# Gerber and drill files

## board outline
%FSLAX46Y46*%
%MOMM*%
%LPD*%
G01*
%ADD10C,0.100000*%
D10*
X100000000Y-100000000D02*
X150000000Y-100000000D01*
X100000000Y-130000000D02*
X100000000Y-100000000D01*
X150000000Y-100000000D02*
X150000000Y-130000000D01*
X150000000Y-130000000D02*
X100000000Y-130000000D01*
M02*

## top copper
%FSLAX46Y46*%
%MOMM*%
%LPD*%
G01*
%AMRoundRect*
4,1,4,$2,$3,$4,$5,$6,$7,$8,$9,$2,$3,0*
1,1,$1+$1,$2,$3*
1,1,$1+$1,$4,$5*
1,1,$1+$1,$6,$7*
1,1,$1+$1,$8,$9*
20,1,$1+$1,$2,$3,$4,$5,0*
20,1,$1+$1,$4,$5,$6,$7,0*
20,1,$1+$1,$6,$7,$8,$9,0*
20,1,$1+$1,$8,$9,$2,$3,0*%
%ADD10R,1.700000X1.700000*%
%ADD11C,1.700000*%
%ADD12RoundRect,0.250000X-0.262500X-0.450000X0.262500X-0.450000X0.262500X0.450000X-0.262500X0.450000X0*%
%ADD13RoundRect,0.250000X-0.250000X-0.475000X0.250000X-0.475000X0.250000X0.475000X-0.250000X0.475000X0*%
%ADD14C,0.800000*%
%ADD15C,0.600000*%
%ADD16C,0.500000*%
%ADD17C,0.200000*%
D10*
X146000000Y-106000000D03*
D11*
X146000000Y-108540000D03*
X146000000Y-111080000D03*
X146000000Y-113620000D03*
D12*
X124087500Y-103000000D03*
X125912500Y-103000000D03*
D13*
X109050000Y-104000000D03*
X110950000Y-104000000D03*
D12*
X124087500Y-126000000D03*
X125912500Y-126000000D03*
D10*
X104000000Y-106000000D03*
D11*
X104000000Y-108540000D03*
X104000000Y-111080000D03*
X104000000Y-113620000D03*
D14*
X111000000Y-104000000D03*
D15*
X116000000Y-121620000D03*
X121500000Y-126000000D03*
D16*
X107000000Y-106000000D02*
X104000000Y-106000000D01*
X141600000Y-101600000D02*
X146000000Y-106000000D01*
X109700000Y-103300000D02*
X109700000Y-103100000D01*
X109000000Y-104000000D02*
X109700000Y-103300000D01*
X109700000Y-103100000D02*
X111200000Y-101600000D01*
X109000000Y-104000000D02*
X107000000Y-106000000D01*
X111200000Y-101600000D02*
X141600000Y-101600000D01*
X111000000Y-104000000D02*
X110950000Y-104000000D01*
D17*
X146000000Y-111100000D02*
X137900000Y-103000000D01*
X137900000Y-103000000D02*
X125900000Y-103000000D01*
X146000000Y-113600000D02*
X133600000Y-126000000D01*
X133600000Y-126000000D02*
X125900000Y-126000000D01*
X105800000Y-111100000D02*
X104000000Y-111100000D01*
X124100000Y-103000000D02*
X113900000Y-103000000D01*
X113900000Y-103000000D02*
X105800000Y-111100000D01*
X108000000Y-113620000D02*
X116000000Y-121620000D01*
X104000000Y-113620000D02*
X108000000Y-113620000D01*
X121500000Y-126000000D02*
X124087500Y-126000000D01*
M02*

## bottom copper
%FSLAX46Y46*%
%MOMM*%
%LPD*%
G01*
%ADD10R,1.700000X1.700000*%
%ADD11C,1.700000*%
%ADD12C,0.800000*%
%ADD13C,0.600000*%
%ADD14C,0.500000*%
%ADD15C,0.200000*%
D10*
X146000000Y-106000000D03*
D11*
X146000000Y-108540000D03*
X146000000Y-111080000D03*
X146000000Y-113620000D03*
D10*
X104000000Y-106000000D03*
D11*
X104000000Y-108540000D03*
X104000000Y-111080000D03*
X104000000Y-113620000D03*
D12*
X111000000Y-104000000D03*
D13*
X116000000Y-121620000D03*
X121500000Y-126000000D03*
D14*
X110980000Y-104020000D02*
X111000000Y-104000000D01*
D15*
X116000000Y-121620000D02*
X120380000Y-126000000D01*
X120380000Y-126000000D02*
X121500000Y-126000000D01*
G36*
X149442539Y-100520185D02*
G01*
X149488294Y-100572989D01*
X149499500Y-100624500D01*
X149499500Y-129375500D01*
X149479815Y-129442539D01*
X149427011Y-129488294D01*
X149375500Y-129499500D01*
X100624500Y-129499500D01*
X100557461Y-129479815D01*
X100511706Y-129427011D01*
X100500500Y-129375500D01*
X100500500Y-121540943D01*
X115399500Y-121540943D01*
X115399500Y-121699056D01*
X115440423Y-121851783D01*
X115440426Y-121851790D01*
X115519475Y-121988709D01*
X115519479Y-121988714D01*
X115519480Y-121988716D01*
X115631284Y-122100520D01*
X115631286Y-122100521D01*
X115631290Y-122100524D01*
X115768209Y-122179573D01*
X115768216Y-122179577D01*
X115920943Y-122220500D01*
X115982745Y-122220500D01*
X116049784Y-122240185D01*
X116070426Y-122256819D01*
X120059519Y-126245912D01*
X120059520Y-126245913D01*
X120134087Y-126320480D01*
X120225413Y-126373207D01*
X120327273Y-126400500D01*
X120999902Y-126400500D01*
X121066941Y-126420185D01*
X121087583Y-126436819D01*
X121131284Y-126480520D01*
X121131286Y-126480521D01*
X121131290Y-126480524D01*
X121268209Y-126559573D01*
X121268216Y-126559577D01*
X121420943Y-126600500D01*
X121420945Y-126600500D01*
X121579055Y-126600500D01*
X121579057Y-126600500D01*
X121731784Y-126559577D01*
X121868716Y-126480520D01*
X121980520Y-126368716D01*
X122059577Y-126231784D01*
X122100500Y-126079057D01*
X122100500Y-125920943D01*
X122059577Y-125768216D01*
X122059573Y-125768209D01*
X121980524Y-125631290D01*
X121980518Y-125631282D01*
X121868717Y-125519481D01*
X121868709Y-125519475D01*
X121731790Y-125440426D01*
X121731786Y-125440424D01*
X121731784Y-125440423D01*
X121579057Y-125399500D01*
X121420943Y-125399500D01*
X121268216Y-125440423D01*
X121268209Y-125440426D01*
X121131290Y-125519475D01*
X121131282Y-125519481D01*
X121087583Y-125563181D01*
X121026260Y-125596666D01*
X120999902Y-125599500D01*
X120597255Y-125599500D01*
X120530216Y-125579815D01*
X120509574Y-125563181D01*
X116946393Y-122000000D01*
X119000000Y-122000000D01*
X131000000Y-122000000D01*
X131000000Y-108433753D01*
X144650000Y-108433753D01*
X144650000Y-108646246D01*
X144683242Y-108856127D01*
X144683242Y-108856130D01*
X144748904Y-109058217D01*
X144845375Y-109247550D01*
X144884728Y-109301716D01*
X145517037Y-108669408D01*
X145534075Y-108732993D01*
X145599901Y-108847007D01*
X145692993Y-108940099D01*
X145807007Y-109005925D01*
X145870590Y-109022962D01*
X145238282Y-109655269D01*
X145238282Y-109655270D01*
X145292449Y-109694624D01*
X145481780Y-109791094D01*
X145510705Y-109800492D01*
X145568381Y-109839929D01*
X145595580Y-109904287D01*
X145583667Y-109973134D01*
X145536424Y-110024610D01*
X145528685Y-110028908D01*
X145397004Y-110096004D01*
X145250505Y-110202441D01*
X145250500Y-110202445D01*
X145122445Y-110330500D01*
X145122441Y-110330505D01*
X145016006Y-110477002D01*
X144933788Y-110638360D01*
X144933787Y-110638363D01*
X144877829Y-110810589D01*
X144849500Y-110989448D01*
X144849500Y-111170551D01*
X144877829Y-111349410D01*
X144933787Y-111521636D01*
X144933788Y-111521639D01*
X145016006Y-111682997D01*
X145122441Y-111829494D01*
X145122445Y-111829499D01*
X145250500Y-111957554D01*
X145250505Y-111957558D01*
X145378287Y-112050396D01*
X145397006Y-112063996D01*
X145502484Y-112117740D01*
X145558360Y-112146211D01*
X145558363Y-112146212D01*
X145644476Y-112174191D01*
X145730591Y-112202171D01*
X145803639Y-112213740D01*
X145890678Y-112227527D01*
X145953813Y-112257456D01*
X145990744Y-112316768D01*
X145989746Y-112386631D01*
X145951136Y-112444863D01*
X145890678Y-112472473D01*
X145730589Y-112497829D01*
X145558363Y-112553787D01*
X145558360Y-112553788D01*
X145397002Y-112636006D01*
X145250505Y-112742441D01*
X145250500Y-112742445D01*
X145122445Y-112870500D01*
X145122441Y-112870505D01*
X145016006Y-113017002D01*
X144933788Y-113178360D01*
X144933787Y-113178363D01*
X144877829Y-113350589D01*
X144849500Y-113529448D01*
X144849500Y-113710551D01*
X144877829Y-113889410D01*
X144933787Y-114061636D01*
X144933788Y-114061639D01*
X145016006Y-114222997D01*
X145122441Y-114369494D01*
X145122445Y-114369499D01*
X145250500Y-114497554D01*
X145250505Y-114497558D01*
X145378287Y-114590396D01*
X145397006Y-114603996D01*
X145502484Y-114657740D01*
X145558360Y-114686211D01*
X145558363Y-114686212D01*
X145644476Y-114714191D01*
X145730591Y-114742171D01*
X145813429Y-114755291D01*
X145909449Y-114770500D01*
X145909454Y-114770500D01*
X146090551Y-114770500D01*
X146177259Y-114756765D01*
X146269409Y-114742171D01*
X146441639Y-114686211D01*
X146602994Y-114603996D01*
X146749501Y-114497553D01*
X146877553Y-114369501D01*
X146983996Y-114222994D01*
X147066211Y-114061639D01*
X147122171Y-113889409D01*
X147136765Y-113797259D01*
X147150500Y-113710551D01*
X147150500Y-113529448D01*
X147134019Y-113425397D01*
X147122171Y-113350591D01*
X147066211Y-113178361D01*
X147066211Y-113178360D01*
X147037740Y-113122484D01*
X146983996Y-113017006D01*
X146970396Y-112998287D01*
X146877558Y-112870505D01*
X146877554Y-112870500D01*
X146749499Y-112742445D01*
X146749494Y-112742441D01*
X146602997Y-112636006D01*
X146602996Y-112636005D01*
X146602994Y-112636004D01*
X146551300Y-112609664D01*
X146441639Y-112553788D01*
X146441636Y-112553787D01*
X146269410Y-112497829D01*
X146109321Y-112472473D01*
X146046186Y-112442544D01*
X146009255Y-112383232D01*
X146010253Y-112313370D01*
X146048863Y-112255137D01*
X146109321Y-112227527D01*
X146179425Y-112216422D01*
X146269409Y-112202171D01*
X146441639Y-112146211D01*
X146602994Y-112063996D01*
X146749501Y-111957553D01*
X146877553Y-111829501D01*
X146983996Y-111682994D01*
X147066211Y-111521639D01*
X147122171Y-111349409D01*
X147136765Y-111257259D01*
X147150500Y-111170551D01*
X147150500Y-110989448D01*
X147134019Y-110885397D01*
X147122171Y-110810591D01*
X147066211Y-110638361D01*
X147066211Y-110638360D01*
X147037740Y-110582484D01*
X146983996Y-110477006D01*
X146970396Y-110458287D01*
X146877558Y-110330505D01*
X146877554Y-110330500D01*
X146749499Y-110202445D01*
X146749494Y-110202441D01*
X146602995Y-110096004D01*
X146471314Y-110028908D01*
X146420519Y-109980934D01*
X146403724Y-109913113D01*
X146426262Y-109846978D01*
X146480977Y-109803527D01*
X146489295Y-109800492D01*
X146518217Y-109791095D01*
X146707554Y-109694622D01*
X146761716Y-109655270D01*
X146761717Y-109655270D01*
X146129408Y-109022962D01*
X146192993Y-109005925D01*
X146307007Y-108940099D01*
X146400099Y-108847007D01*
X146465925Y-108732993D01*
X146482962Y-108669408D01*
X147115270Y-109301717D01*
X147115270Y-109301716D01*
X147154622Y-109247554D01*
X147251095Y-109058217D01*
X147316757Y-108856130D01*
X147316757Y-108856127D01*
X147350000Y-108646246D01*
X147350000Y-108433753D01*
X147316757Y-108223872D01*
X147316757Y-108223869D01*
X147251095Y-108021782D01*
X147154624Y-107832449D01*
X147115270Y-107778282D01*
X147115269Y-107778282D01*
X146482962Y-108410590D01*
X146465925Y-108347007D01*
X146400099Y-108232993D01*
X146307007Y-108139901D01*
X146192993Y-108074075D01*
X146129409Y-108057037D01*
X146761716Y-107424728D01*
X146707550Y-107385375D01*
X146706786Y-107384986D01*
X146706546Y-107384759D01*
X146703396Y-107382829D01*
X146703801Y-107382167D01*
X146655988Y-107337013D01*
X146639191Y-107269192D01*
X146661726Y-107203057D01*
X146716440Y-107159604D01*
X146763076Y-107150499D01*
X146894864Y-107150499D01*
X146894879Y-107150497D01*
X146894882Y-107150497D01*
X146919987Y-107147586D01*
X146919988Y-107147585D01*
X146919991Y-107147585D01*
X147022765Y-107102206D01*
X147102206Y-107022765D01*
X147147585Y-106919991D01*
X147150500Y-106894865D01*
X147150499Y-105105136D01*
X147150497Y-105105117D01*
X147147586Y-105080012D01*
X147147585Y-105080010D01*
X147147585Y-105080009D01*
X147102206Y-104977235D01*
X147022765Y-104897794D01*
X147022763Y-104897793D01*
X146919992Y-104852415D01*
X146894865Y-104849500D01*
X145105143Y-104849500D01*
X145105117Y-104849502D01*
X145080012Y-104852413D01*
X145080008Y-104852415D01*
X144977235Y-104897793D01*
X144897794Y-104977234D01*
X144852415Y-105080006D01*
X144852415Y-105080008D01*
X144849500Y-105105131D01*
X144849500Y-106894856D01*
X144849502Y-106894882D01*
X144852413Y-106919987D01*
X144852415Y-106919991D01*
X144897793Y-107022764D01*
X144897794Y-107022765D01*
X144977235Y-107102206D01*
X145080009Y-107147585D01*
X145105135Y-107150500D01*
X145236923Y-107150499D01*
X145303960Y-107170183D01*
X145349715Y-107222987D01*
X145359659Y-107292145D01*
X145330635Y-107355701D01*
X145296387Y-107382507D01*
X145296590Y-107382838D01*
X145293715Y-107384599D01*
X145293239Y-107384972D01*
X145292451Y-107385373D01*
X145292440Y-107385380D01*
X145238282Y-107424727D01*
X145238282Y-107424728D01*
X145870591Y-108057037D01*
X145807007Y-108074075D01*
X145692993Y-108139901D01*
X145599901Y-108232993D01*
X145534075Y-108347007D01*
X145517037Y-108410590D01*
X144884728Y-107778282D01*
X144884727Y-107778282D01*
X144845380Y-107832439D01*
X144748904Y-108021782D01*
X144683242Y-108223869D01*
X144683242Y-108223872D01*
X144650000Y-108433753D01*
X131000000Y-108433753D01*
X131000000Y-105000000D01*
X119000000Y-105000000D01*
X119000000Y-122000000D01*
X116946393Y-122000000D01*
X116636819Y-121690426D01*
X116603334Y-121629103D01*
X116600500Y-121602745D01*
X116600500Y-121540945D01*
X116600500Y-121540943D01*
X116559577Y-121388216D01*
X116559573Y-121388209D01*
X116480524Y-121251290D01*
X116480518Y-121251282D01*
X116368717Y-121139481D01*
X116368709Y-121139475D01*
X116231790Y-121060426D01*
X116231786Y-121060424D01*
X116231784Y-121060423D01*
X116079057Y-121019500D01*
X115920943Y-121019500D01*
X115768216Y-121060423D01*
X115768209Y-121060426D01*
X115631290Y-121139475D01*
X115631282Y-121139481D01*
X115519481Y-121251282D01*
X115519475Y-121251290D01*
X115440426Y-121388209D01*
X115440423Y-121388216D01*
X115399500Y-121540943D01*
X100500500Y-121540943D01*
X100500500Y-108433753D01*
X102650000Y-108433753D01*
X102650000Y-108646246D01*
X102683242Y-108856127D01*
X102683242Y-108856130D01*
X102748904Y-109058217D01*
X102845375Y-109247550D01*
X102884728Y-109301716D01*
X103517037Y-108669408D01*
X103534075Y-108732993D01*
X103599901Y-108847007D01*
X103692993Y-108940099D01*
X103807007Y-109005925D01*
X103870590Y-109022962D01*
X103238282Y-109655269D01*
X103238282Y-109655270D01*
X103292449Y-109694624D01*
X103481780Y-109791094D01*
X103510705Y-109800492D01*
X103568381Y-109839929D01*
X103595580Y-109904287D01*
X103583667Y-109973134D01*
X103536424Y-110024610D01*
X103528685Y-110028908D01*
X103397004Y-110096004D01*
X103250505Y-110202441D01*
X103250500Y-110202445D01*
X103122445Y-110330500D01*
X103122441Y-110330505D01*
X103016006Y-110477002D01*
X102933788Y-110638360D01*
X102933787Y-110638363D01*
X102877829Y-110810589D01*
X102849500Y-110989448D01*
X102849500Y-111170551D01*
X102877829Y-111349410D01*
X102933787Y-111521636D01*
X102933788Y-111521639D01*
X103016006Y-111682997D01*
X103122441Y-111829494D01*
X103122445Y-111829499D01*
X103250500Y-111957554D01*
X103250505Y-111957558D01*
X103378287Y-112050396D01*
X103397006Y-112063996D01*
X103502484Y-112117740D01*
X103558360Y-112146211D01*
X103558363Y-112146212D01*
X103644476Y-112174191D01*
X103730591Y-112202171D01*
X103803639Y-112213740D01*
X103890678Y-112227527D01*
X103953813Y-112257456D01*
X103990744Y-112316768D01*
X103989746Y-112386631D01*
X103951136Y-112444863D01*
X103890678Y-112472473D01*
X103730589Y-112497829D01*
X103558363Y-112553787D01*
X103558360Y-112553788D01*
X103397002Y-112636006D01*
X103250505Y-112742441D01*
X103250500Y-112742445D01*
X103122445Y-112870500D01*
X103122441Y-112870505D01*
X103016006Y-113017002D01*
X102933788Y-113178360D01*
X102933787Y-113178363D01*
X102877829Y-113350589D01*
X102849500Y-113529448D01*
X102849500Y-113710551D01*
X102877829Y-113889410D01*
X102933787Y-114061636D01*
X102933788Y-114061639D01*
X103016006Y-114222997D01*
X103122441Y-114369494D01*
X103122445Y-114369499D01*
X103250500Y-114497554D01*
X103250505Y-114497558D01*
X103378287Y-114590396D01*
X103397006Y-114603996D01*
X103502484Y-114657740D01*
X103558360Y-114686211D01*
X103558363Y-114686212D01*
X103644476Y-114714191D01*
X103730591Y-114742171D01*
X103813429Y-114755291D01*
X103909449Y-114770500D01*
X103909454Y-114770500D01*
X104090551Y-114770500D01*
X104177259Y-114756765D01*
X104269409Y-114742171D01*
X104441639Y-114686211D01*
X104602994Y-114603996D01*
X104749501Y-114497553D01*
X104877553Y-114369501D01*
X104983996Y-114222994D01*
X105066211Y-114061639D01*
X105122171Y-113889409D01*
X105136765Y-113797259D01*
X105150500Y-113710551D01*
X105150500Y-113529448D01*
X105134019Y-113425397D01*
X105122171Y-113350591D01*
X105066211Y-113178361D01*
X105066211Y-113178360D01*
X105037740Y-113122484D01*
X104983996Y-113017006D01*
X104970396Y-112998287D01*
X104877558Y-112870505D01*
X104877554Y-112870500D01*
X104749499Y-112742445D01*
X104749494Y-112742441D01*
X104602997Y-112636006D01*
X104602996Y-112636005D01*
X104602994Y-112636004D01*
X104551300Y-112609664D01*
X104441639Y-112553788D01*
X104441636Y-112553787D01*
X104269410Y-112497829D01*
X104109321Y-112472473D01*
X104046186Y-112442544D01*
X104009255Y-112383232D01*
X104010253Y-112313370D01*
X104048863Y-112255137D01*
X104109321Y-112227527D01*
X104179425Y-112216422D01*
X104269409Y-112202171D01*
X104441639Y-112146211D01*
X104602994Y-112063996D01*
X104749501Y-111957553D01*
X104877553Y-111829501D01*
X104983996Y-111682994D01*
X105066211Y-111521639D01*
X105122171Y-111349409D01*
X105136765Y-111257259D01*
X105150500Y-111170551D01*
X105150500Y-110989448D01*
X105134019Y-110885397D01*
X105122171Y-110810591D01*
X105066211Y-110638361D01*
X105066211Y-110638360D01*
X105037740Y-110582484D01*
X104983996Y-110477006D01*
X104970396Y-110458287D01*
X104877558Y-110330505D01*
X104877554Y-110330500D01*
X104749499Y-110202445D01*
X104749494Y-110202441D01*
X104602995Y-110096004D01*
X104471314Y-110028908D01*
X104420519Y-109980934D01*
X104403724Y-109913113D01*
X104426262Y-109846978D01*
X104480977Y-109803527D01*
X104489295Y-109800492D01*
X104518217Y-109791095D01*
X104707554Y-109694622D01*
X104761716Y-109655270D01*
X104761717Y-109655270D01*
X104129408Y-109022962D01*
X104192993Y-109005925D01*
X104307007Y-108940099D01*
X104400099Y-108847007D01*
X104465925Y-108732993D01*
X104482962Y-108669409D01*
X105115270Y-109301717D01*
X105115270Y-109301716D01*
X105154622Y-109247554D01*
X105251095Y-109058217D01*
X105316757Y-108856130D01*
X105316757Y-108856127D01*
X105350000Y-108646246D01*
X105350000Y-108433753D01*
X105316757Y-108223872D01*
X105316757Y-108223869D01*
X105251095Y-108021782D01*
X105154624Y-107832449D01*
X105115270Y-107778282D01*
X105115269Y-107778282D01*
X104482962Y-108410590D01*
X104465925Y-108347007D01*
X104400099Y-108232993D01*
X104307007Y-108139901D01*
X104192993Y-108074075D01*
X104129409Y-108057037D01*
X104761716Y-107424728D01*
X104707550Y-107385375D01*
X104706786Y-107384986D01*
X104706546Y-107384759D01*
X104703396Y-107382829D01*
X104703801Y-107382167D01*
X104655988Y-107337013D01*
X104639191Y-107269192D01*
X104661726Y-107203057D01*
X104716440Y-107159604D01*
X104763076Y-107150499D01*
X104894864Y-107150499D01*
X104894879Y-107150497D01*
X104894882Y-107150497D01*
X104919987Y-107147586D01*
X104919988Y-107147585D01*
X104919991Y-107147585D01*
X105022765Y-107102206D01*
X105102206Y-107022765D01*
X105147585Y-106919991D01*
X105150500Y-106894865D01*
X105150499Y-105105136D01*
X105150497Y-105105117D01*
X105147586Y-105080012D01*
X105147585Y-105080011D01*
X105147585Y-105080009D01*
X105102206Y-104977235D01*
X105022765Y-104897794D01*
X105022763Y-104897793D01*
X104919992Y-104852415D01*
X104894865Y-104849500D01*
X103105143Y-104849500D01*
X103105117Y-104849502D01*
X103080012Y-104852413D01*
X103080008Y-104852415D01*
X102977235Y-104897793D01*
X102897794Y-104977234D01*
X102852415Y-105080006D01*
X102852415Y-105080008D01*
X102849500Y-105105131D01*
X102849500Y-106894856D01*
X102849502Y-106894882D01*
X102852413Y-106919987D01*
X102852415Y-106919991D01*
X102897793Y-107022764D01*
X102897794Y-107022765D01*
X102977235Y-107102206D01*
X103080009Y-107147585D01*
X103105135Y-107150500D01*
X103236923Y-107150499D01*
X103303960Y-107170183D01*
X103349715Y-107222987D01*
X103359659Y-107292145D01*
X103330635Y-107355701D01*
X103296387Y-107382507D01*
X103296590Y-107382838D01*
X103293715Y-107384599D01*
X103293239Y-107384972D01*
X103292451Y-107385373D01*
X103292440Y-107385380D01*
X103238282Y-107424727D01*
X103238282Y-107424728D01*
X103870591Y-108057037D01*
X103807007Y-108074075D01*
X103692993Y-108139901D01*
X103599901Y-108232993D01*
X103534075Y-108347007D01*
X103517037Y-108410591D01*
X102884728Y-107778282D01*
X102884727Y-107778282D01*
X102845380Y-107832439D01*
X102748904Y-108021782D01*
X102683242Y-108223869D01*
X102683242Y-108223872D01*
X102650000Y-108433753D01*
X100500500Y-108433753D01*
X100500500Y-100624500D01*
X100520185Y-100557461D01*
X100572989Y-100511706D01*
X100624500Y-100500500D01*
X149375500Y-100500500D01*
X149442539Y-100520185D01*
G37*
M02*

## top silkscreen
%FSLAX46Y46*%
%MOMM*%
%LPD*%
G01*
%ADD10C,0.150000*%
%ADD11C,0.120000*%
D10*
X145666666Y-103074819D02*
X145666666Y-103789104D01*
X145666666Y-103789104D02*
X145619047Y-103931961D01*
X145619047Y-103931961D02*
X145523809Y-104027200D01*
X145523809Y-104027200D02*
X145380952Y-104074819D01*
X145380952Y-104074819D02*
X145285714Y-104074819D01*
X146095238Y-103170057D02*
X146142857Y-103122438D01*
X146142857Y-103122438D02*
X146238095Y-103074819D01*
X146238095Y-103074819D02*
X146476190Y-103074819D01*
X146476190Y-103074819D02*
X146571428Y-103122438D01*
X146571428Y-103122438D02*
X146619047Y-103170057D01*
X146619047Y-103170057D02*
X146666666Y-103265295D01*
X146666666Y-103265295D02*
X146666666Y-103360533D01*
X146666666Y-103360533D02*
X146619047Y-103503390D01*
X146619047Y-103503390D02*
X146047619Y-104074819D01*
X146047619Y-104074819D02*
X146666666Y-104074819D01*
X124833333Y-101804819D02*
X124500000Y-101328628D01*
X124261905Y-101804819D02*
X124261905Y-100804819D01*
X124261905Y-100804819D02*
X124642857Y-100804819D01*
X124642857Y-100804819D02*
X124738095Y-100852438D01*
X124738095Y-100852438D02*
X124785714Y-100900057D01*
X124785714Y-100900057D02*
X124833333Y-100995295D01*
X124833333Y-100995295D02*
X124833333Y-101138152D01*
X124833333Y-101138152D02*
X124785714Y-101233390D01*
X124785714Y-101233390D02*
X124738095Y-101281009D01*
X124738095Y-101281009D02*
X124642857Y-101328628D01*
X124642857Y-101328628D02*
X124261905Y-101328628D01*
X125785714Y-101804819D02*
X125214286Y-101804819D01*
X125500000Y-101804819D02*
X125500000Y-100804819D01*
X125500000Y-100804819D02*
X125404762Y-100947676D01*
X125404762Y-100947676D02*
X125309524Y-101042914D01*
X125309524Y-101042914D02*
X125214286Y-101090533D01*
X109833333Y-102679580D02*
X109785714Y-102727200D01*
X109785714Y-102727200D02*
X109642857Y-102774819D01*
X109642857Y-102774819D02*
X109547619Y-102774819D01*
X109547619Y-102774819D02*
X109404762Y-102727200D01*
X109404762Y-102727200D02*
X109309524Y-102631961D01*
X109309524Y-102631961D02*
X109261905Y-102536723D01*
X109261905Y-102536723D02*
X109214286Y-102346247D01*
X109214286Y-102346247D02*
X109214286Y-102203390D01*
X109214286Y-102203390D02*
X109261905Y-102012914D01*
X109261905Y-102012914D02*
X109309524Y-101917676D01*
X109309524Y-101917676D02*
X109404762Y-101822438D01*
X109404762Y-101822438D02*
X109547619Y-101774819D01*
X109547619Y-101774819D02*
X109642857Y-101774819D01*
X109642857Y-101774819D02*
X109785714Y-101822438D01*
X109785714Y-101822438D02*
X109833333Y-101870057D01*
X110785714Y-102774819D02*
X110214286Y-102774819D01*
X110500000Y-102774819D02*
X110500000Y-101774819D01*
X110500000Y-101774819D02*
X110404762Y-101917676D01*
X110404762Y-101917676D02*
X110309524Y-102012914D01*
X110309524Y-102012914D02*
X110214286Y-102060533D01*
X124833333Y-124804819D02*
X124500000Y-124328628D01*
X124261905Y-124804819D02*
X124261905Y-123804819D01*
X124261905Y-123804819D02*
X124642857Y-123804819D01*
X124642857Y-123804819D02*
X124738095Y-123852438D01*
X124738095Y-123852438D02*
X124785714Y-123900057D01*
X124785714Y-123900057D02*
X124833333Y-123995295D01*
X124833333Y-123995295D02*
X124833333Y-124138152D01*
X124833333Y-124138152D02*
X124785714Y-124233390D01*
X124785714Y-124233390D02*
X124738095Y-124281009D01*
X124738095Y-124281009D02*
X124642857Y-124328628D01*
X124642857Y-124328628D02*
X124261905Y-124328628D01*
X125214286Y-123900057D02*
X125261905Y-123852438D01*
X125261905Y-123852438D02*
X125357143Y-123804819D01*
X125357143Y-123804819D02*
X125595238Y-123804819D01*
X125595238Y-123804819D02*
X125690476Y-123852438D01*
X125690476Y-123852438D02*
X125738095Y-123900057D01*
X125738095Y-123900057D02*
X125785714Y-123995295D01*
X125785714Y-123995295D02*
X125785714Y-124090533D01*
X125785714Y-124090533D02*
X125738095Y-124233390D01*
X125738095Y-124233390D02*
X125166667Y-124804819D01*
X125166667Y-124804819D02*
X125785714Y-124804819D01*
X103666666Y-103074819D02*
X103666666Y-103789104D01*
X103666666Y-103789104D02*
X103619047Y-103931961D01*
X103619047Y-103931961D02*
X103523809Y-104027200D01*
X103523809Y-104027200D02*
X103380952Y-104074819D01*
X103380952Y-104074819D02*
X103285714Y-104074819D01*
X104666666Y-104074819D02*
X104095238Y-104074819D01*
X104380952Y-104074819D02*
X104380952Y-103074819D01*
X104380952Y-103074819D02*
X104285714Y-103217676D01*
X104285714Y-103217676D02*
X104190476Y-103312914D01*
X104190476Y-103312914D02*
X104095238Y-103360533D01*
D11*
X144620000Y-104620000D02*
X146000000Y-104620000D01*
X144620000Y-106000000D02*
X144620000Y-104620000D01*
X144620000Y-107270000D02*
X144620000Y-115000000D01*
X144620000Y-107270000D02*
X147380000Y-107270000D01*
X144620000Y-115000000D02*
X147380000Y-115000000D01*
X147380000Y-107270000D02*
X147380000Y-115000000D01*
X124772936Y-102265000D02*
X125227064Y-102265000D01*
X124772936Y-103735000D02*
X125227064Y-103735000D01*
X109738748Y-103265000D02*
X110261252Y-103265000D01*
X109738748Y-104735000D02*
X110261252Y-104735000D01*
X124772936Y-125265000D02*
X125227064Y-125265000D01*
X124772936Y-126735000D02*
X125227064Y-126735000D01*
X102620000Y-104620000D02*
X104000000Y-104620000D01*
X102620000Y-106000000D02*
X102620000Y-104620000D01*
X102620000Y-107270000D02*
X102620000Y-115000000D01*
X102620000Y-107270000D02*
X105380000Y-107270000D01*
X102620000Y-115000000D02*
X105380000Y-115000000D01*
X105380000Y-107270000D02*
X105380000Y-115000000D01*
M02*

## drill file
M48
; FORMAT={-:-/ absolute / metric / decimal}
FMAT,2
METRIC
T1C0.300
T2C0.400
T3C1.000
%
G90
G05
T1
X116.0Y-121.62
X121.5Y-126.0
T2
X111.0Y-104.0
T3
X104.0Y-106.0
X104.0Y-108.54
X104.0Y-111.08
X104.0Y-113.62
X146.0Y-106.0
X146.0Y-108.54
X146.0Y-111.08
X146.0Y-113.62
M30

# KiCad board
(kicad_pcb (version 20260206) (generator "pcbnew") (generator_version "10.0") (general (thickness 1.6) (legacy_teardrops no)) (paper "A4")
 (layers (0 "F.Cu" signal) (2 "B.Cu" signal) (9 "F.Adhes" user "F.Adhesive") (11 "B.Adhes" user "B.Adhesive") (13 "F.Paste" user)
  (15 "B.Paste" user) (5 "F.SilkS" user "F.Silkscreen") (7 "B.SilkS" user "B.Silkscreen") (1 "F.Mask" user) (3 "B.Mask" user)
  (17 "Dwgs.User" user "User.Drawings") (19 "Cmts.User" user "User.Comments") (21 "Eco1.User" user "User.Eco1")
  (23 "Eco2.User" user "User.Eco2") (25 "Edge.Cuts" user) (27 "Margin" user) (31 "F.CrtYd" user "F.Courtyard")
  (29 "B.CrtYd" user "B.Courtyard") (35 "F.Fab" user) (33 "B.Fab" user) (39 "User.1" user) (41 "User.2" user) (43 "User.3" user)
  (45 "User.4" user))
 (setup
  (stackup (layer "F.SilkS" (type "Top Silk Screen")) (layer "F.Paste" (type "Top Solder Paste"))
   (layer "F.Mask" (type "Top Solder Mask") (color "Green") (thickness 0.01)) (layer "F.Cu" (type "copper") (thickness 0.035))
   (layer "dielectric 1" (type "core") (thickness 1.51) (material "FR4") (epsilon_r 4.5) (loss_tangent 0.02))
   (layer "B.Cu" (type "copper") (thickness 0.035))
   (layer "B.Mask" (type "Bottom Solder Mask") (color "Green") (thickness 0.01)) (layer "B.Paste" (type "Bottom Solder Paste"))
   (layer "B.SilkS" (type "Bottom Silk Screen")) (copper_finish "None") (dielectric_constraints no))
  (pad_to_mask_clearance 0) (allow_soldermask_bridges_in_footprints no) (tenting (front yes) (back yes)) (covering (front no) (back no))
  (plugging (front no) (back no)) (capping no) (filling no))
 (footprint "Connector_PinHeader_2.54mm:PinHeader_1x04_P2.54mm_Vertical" (layer "F.Cu") (at 146 106)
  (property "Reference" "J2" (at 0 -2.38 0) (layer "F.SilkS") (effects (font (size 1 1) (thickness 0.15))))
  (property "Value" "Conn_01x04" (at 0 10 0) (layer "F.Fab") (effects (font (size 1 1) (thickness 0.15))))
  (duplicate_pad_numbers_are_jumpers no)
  (fp_line (start -1.38 -1.38) (end 0 -1.38) (stroke (width 0.12) (type solid)) (layer "F.SilkS"))
  (fp_line (start -1.38 0) (end -1.38 -1.38) (stroke (width 0.12) (type solid)) (layer "F.SilkS"))
  (fp_line (start -1.38 1.27) (end -1.38 9) (stroke (width 0.12) (type solid)) (layer "F.SilkS"))
  (fp_line (start -1.38 1.27) (end 1.38 1.27) (stroke (width 0.12) (type solid)) (layer "F.SilkS"))
  (fp_line (start -1.38 9) (end 1.38 9) (stroke (width 0.12) (type solid)) (layer "F.SilkS"))
  (fp_line (start 1.38 1.27) (end 1.38 9) (stroke (width 0.12) (type solid)) (layer "F.SilkS"))
  (pad "1" thru_hole rect (at 0 0) (size 1.7 1.7) (drill 1) (layers "*.Cu" "*.Mask") (remove_unused_layers no) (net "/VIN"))
  (pad "2" thru_hole circle (at 0 2.54) (size 1.7 1.7) (drill 1) (layers "*.Cu" "*.Mask") (remove_unused_layers no) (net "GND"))
  (pad "3" thru_hole circle (at 0 5.08) (size 1.7 1.7) (drill 1) (layers "*.Cu" "*.Mask") (remove_unused_layers no) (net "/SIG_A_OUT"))
  (pad "4" thru_hole circle (at 0 7.62) (size 1.7 1.7) (drill 1) (layers "*.Cu" "*.Mask") (remove_unused_layers no) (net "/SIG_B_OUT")))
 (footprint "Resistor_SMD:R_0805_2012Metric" (layer "F.Cu") (at 125 103)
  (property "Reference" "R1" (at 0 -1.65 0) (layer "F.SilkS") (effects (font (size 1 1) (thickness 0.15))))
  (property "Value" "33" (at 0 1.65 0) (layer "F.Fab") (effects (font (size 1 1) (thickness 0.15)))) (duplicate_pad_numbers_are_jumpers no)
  (fp_line (start -0.227064 -0.735) (end 0.227064 -0.735) (stroke (width 0.12) (type solid)) (layer "F.SilkS"))
  (fp_line (start -0.227064 0.735) (end 0.227064 0.735) (stroke (width 0.12) (type solid)) (layer "F.SilkS"))
  (pad "1" smd roundrect (at -0.9125 0) (size 1.025 1.4) (layers "F.Cu" "F.Mask" "F.Paste") (roundrect_rratio 0.243902) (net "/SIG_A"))
  (pad "2" smd roundrect (at 0.9125 0) (size 1.025 1.4) (layers "F.Cu" "F.Mask" "F.Paste") (roundrect_rratio 0.243902) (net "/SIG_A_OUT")))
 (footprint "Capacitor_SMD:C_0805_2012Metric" (layer "F.Cu") (at 110 104)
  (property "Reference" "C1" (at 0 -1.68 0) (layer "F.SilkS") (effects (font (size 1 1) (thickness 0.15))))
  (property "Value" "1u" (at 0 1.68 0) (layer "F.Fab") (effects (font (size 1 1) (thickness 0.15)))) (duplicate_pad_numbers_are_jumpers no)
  (fp_line (start -0.261252 -0.735) (end 0.261252 -0.735) (stroke (width 0.12) (type solid)) (layer "F.SilkS"))
  (fp_line (start -0.261252 0.735) (end 0.261252 0.735) (stroke (width 0.12) (type solid)) (layer "F.SilkS"))
  (pad "1" smd roundrect (at -0.95 0) (size 1 1.45) (layers "F.Cu" "F.Mask" "F.Paste") (roundrect_rratio 0.25) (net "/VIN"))
  (pad "2" smd roundrect (at 0.95 0) (size 1 1.45) (layers "F.Cu" "F.Mask" "F.Paste") (roundrect_rratio 0.25) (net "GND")))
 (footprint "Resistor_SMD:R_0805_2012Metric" (layer "F.Cu") (at 125 126)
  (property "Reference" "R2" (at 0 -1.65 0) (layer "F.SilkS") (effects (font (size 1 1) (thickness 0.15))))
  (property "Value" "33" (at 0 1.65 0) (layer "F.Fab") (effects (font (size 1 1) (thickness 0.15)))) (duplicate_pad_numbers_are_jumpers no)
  (fp_line (start -0.227064 -0.735) (end 0.227064 -0.735) (stroke (width 0.12) (type solid)) (layer "F.SilkS"))
  (fp_line (start -0.227064 0.735) (end 0.227064 0.735) (stroke (width 0.12) (type solid)) (layer "F.SilkS"))
  (pad "1" smd roundrect (at -0.9125 0) (size 1.025 1.4) (layers "F.Cu" "F.Mask" "F.Paste") (roundrect_rratio 0.243902) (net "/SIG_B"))
  (pad "2" smd roundrect (at 0.9125 0) (size 1.025 1.4) (layers "F.Cu" "F.Mask" "F.Paste") (roundrect_rratio 0.243902) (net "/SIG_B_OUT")))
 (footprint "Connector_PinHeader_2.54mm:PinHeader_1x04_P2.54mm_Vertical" (layer "F.Cu") (at 104 106)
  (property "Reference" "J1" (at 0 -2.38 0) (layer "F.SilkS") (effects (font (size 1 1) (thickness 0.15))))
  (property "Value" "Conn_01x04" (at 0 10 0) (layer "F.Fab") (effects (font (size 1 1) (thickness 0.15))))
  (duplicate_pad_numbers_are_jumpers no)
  (fp_line (start -1.38 -1.38) (end 0 -1.38) (stroke (width 0.12) (type solid)) (layer "F.SilkS"))
  (fp_line (start -1.38 0) (end -1.38 -1.38) (stroke (width 0.12) (type solid)) (layer "F.SilkS"))
  (fp_line (start -1.38 1.27) (end -1.38 9) (stroke (width 0.12) (type solid)) (layer "F.SilkS"))
  (fp_line (start -1.38 1.27) (end 1.38 1.27) (stroke (width 0.12) (type solid)) (layer "F.SilkS"))
  (fp_line (start -1.38 9) (end 1.38 9) (stroke (width 0.12) (type solid)) (layer "F.SilkS"))
  (fp_line (start 1.38 1.27) (end 1.38 9) (stroke (width 0.12) (type solid)) (layer "F.SilkS"))
  (pad "1" thru_hole rect (at 0 0) (size 1.7 1.7) (drill 1) (layers "*.Cu" "*.Mask") (remove_unused_layers no) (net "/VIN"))
  (pad "2" thru_hole circle (at 0 2.54) (size 1.7 1.7) (drill 1) (layers "*.Cu" "*.Mask") (remove_unused_layers no) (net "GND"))
  (pad "3" thru_hole circle (at 0 5.08) (size 1.7 1.7) (drill 1) (layers "*.Cu" "*.Mask") (remove_unused_layers no) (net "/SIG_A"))
  (pad "4" thru_hole circle (at 0 7.62) (size 1.7 1.7) (drill 1) (layers "*.Cu" "*.Mask") (remove_unused_layers no) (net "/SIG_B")))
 (gr_line (start 100 100) (end 150 100) (stroke (width 0.1) (type default)) (layer "Edge.Cuts"))
 (gr_line (start 100 130) (end 100 100) (stroke (width 0.1) (type default)) (layer "Edge.Cuts"))
 (gr_line (start 150 100) (end 150 130) (stroke (width 0.1) (type default)) (layer "Edge.Cuts"))
 (gr_line (start 150 130) (end 100 130) (stroke (width 0.1) (type default)) (layer "Edge.Cuts"))
 (segment (start 107 106) (end 104 106) (width 0.5) (layer "F.Cu") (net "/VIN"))
 (segment (start 141.6 101.6) (end 146 106) (width 0.5) (layer "F.Cu") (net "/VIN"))
 (segment (start 109.7 103.3) (end 109.7 103.1) (width 0.5) (layer "F.Cu") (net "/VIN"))
 (segment (start 109 104) (end 109.7 103.3) (width 0.5) (layer "F.Cu") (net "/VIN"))
 (segment (start 109.7 103.1) (end 111.2 101.6) (width 0.5) (layer "F.Cu") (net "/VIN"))
 (segment (start 109 104) (end 107 106) (width 0.5) (layer "F.Cu") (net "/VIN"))
 (segment (start 111.2 101.6) (end 141.6 101.6) (width 0.5) (layer "F.Cu") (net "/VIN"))
 (segment (start 111 104) (end 110.95 104) (width 0.5) (layer "F.Cu") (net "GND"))
 (via (at 111 104) (size 0.8) (drill 0.4) (layers "F.Cu" "B.Cu") (capping yes) (filling yes) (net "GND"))
 (segment (start 110.98 104.02) (end 111 104) (width 0.5) (layer "B.Cu") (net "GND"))
 (segment (start 146 111.1) (end 137.9 103) (width 0.2) (layer "F.Cu") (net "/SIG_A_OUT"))
 (segment (start 137.9 103) (end 125.9 103) (width 0.2) (layer "F.Cu") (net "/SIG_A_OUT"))
 (segment (start 146 113.6) (end 133.6 126) (width 0.2) (layer "F.Cu") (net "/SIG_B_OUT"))
 (segment (start 133.6 126) (end 125.9 126) (width 0.2) (layer "F.Cu") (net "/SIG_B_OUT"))
 (segment (start 105.8 111.1) (end 104 111.1) (width 0.2) (layer "F.Cu") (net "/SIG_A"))
 (segment (start 124.1 103) (end 113.9 103) (width 0.2) (layer "F.Cu") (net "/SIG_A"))
 (segment (start 113.9 103) (end 105.8 111.1) (width 0.2) (layer "F.Cu") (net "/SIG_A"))
 (segment (start 108 113.62) (end 116 121.62) (width 0.2) (locked yes) (layer "F.Cu") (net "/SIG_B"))
 (segment (start 104 113.62) (end 108 113.62) (width 0.2) (locked yes) (layer "F.Cu") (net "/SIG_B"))
 (segment (start 121.5 126) (end 124.0875 126) (width 0.2) (locked yes) (layer "F.Cu") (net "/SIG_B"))
 (via (at 116 121.62) (size 0.6) (drill 0.3) (layers "F.Cu" "B.Cu") (locked yes) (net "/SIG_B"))
 (via (at 121.5 126) (size 0.6) (drill 0.3) (layers "F.Cu" "B.Cu") (locked yes) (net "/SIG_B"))
 (segment (start 116 121.62) (end 120.38 126) (width 0.2) (locked yes) (layer "B.Cu") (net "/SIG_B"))
 (segment (start 120.38 126) (end 121.5 126) (width 0.2) (locked yes) (layer "B.Cu") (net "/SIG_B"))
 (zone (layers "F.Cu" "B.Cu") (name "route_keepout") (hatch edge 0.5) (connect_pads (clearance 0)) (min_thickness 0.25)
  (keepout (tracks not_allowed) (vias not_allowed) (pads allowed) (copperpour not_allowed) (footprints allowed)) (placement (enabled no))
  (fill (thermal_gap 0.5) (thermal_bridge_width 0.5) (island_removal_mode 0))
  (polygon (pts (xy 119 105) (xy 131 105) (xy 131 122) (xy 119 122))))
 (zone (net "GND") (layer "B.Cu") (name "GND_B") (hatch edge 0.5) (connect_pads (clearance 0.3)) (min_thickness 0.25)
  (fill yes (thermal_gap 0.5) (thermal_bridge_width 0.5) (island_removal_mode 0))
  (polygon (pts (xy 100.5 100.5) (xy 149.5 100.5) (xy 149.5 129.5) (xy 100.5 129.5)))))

